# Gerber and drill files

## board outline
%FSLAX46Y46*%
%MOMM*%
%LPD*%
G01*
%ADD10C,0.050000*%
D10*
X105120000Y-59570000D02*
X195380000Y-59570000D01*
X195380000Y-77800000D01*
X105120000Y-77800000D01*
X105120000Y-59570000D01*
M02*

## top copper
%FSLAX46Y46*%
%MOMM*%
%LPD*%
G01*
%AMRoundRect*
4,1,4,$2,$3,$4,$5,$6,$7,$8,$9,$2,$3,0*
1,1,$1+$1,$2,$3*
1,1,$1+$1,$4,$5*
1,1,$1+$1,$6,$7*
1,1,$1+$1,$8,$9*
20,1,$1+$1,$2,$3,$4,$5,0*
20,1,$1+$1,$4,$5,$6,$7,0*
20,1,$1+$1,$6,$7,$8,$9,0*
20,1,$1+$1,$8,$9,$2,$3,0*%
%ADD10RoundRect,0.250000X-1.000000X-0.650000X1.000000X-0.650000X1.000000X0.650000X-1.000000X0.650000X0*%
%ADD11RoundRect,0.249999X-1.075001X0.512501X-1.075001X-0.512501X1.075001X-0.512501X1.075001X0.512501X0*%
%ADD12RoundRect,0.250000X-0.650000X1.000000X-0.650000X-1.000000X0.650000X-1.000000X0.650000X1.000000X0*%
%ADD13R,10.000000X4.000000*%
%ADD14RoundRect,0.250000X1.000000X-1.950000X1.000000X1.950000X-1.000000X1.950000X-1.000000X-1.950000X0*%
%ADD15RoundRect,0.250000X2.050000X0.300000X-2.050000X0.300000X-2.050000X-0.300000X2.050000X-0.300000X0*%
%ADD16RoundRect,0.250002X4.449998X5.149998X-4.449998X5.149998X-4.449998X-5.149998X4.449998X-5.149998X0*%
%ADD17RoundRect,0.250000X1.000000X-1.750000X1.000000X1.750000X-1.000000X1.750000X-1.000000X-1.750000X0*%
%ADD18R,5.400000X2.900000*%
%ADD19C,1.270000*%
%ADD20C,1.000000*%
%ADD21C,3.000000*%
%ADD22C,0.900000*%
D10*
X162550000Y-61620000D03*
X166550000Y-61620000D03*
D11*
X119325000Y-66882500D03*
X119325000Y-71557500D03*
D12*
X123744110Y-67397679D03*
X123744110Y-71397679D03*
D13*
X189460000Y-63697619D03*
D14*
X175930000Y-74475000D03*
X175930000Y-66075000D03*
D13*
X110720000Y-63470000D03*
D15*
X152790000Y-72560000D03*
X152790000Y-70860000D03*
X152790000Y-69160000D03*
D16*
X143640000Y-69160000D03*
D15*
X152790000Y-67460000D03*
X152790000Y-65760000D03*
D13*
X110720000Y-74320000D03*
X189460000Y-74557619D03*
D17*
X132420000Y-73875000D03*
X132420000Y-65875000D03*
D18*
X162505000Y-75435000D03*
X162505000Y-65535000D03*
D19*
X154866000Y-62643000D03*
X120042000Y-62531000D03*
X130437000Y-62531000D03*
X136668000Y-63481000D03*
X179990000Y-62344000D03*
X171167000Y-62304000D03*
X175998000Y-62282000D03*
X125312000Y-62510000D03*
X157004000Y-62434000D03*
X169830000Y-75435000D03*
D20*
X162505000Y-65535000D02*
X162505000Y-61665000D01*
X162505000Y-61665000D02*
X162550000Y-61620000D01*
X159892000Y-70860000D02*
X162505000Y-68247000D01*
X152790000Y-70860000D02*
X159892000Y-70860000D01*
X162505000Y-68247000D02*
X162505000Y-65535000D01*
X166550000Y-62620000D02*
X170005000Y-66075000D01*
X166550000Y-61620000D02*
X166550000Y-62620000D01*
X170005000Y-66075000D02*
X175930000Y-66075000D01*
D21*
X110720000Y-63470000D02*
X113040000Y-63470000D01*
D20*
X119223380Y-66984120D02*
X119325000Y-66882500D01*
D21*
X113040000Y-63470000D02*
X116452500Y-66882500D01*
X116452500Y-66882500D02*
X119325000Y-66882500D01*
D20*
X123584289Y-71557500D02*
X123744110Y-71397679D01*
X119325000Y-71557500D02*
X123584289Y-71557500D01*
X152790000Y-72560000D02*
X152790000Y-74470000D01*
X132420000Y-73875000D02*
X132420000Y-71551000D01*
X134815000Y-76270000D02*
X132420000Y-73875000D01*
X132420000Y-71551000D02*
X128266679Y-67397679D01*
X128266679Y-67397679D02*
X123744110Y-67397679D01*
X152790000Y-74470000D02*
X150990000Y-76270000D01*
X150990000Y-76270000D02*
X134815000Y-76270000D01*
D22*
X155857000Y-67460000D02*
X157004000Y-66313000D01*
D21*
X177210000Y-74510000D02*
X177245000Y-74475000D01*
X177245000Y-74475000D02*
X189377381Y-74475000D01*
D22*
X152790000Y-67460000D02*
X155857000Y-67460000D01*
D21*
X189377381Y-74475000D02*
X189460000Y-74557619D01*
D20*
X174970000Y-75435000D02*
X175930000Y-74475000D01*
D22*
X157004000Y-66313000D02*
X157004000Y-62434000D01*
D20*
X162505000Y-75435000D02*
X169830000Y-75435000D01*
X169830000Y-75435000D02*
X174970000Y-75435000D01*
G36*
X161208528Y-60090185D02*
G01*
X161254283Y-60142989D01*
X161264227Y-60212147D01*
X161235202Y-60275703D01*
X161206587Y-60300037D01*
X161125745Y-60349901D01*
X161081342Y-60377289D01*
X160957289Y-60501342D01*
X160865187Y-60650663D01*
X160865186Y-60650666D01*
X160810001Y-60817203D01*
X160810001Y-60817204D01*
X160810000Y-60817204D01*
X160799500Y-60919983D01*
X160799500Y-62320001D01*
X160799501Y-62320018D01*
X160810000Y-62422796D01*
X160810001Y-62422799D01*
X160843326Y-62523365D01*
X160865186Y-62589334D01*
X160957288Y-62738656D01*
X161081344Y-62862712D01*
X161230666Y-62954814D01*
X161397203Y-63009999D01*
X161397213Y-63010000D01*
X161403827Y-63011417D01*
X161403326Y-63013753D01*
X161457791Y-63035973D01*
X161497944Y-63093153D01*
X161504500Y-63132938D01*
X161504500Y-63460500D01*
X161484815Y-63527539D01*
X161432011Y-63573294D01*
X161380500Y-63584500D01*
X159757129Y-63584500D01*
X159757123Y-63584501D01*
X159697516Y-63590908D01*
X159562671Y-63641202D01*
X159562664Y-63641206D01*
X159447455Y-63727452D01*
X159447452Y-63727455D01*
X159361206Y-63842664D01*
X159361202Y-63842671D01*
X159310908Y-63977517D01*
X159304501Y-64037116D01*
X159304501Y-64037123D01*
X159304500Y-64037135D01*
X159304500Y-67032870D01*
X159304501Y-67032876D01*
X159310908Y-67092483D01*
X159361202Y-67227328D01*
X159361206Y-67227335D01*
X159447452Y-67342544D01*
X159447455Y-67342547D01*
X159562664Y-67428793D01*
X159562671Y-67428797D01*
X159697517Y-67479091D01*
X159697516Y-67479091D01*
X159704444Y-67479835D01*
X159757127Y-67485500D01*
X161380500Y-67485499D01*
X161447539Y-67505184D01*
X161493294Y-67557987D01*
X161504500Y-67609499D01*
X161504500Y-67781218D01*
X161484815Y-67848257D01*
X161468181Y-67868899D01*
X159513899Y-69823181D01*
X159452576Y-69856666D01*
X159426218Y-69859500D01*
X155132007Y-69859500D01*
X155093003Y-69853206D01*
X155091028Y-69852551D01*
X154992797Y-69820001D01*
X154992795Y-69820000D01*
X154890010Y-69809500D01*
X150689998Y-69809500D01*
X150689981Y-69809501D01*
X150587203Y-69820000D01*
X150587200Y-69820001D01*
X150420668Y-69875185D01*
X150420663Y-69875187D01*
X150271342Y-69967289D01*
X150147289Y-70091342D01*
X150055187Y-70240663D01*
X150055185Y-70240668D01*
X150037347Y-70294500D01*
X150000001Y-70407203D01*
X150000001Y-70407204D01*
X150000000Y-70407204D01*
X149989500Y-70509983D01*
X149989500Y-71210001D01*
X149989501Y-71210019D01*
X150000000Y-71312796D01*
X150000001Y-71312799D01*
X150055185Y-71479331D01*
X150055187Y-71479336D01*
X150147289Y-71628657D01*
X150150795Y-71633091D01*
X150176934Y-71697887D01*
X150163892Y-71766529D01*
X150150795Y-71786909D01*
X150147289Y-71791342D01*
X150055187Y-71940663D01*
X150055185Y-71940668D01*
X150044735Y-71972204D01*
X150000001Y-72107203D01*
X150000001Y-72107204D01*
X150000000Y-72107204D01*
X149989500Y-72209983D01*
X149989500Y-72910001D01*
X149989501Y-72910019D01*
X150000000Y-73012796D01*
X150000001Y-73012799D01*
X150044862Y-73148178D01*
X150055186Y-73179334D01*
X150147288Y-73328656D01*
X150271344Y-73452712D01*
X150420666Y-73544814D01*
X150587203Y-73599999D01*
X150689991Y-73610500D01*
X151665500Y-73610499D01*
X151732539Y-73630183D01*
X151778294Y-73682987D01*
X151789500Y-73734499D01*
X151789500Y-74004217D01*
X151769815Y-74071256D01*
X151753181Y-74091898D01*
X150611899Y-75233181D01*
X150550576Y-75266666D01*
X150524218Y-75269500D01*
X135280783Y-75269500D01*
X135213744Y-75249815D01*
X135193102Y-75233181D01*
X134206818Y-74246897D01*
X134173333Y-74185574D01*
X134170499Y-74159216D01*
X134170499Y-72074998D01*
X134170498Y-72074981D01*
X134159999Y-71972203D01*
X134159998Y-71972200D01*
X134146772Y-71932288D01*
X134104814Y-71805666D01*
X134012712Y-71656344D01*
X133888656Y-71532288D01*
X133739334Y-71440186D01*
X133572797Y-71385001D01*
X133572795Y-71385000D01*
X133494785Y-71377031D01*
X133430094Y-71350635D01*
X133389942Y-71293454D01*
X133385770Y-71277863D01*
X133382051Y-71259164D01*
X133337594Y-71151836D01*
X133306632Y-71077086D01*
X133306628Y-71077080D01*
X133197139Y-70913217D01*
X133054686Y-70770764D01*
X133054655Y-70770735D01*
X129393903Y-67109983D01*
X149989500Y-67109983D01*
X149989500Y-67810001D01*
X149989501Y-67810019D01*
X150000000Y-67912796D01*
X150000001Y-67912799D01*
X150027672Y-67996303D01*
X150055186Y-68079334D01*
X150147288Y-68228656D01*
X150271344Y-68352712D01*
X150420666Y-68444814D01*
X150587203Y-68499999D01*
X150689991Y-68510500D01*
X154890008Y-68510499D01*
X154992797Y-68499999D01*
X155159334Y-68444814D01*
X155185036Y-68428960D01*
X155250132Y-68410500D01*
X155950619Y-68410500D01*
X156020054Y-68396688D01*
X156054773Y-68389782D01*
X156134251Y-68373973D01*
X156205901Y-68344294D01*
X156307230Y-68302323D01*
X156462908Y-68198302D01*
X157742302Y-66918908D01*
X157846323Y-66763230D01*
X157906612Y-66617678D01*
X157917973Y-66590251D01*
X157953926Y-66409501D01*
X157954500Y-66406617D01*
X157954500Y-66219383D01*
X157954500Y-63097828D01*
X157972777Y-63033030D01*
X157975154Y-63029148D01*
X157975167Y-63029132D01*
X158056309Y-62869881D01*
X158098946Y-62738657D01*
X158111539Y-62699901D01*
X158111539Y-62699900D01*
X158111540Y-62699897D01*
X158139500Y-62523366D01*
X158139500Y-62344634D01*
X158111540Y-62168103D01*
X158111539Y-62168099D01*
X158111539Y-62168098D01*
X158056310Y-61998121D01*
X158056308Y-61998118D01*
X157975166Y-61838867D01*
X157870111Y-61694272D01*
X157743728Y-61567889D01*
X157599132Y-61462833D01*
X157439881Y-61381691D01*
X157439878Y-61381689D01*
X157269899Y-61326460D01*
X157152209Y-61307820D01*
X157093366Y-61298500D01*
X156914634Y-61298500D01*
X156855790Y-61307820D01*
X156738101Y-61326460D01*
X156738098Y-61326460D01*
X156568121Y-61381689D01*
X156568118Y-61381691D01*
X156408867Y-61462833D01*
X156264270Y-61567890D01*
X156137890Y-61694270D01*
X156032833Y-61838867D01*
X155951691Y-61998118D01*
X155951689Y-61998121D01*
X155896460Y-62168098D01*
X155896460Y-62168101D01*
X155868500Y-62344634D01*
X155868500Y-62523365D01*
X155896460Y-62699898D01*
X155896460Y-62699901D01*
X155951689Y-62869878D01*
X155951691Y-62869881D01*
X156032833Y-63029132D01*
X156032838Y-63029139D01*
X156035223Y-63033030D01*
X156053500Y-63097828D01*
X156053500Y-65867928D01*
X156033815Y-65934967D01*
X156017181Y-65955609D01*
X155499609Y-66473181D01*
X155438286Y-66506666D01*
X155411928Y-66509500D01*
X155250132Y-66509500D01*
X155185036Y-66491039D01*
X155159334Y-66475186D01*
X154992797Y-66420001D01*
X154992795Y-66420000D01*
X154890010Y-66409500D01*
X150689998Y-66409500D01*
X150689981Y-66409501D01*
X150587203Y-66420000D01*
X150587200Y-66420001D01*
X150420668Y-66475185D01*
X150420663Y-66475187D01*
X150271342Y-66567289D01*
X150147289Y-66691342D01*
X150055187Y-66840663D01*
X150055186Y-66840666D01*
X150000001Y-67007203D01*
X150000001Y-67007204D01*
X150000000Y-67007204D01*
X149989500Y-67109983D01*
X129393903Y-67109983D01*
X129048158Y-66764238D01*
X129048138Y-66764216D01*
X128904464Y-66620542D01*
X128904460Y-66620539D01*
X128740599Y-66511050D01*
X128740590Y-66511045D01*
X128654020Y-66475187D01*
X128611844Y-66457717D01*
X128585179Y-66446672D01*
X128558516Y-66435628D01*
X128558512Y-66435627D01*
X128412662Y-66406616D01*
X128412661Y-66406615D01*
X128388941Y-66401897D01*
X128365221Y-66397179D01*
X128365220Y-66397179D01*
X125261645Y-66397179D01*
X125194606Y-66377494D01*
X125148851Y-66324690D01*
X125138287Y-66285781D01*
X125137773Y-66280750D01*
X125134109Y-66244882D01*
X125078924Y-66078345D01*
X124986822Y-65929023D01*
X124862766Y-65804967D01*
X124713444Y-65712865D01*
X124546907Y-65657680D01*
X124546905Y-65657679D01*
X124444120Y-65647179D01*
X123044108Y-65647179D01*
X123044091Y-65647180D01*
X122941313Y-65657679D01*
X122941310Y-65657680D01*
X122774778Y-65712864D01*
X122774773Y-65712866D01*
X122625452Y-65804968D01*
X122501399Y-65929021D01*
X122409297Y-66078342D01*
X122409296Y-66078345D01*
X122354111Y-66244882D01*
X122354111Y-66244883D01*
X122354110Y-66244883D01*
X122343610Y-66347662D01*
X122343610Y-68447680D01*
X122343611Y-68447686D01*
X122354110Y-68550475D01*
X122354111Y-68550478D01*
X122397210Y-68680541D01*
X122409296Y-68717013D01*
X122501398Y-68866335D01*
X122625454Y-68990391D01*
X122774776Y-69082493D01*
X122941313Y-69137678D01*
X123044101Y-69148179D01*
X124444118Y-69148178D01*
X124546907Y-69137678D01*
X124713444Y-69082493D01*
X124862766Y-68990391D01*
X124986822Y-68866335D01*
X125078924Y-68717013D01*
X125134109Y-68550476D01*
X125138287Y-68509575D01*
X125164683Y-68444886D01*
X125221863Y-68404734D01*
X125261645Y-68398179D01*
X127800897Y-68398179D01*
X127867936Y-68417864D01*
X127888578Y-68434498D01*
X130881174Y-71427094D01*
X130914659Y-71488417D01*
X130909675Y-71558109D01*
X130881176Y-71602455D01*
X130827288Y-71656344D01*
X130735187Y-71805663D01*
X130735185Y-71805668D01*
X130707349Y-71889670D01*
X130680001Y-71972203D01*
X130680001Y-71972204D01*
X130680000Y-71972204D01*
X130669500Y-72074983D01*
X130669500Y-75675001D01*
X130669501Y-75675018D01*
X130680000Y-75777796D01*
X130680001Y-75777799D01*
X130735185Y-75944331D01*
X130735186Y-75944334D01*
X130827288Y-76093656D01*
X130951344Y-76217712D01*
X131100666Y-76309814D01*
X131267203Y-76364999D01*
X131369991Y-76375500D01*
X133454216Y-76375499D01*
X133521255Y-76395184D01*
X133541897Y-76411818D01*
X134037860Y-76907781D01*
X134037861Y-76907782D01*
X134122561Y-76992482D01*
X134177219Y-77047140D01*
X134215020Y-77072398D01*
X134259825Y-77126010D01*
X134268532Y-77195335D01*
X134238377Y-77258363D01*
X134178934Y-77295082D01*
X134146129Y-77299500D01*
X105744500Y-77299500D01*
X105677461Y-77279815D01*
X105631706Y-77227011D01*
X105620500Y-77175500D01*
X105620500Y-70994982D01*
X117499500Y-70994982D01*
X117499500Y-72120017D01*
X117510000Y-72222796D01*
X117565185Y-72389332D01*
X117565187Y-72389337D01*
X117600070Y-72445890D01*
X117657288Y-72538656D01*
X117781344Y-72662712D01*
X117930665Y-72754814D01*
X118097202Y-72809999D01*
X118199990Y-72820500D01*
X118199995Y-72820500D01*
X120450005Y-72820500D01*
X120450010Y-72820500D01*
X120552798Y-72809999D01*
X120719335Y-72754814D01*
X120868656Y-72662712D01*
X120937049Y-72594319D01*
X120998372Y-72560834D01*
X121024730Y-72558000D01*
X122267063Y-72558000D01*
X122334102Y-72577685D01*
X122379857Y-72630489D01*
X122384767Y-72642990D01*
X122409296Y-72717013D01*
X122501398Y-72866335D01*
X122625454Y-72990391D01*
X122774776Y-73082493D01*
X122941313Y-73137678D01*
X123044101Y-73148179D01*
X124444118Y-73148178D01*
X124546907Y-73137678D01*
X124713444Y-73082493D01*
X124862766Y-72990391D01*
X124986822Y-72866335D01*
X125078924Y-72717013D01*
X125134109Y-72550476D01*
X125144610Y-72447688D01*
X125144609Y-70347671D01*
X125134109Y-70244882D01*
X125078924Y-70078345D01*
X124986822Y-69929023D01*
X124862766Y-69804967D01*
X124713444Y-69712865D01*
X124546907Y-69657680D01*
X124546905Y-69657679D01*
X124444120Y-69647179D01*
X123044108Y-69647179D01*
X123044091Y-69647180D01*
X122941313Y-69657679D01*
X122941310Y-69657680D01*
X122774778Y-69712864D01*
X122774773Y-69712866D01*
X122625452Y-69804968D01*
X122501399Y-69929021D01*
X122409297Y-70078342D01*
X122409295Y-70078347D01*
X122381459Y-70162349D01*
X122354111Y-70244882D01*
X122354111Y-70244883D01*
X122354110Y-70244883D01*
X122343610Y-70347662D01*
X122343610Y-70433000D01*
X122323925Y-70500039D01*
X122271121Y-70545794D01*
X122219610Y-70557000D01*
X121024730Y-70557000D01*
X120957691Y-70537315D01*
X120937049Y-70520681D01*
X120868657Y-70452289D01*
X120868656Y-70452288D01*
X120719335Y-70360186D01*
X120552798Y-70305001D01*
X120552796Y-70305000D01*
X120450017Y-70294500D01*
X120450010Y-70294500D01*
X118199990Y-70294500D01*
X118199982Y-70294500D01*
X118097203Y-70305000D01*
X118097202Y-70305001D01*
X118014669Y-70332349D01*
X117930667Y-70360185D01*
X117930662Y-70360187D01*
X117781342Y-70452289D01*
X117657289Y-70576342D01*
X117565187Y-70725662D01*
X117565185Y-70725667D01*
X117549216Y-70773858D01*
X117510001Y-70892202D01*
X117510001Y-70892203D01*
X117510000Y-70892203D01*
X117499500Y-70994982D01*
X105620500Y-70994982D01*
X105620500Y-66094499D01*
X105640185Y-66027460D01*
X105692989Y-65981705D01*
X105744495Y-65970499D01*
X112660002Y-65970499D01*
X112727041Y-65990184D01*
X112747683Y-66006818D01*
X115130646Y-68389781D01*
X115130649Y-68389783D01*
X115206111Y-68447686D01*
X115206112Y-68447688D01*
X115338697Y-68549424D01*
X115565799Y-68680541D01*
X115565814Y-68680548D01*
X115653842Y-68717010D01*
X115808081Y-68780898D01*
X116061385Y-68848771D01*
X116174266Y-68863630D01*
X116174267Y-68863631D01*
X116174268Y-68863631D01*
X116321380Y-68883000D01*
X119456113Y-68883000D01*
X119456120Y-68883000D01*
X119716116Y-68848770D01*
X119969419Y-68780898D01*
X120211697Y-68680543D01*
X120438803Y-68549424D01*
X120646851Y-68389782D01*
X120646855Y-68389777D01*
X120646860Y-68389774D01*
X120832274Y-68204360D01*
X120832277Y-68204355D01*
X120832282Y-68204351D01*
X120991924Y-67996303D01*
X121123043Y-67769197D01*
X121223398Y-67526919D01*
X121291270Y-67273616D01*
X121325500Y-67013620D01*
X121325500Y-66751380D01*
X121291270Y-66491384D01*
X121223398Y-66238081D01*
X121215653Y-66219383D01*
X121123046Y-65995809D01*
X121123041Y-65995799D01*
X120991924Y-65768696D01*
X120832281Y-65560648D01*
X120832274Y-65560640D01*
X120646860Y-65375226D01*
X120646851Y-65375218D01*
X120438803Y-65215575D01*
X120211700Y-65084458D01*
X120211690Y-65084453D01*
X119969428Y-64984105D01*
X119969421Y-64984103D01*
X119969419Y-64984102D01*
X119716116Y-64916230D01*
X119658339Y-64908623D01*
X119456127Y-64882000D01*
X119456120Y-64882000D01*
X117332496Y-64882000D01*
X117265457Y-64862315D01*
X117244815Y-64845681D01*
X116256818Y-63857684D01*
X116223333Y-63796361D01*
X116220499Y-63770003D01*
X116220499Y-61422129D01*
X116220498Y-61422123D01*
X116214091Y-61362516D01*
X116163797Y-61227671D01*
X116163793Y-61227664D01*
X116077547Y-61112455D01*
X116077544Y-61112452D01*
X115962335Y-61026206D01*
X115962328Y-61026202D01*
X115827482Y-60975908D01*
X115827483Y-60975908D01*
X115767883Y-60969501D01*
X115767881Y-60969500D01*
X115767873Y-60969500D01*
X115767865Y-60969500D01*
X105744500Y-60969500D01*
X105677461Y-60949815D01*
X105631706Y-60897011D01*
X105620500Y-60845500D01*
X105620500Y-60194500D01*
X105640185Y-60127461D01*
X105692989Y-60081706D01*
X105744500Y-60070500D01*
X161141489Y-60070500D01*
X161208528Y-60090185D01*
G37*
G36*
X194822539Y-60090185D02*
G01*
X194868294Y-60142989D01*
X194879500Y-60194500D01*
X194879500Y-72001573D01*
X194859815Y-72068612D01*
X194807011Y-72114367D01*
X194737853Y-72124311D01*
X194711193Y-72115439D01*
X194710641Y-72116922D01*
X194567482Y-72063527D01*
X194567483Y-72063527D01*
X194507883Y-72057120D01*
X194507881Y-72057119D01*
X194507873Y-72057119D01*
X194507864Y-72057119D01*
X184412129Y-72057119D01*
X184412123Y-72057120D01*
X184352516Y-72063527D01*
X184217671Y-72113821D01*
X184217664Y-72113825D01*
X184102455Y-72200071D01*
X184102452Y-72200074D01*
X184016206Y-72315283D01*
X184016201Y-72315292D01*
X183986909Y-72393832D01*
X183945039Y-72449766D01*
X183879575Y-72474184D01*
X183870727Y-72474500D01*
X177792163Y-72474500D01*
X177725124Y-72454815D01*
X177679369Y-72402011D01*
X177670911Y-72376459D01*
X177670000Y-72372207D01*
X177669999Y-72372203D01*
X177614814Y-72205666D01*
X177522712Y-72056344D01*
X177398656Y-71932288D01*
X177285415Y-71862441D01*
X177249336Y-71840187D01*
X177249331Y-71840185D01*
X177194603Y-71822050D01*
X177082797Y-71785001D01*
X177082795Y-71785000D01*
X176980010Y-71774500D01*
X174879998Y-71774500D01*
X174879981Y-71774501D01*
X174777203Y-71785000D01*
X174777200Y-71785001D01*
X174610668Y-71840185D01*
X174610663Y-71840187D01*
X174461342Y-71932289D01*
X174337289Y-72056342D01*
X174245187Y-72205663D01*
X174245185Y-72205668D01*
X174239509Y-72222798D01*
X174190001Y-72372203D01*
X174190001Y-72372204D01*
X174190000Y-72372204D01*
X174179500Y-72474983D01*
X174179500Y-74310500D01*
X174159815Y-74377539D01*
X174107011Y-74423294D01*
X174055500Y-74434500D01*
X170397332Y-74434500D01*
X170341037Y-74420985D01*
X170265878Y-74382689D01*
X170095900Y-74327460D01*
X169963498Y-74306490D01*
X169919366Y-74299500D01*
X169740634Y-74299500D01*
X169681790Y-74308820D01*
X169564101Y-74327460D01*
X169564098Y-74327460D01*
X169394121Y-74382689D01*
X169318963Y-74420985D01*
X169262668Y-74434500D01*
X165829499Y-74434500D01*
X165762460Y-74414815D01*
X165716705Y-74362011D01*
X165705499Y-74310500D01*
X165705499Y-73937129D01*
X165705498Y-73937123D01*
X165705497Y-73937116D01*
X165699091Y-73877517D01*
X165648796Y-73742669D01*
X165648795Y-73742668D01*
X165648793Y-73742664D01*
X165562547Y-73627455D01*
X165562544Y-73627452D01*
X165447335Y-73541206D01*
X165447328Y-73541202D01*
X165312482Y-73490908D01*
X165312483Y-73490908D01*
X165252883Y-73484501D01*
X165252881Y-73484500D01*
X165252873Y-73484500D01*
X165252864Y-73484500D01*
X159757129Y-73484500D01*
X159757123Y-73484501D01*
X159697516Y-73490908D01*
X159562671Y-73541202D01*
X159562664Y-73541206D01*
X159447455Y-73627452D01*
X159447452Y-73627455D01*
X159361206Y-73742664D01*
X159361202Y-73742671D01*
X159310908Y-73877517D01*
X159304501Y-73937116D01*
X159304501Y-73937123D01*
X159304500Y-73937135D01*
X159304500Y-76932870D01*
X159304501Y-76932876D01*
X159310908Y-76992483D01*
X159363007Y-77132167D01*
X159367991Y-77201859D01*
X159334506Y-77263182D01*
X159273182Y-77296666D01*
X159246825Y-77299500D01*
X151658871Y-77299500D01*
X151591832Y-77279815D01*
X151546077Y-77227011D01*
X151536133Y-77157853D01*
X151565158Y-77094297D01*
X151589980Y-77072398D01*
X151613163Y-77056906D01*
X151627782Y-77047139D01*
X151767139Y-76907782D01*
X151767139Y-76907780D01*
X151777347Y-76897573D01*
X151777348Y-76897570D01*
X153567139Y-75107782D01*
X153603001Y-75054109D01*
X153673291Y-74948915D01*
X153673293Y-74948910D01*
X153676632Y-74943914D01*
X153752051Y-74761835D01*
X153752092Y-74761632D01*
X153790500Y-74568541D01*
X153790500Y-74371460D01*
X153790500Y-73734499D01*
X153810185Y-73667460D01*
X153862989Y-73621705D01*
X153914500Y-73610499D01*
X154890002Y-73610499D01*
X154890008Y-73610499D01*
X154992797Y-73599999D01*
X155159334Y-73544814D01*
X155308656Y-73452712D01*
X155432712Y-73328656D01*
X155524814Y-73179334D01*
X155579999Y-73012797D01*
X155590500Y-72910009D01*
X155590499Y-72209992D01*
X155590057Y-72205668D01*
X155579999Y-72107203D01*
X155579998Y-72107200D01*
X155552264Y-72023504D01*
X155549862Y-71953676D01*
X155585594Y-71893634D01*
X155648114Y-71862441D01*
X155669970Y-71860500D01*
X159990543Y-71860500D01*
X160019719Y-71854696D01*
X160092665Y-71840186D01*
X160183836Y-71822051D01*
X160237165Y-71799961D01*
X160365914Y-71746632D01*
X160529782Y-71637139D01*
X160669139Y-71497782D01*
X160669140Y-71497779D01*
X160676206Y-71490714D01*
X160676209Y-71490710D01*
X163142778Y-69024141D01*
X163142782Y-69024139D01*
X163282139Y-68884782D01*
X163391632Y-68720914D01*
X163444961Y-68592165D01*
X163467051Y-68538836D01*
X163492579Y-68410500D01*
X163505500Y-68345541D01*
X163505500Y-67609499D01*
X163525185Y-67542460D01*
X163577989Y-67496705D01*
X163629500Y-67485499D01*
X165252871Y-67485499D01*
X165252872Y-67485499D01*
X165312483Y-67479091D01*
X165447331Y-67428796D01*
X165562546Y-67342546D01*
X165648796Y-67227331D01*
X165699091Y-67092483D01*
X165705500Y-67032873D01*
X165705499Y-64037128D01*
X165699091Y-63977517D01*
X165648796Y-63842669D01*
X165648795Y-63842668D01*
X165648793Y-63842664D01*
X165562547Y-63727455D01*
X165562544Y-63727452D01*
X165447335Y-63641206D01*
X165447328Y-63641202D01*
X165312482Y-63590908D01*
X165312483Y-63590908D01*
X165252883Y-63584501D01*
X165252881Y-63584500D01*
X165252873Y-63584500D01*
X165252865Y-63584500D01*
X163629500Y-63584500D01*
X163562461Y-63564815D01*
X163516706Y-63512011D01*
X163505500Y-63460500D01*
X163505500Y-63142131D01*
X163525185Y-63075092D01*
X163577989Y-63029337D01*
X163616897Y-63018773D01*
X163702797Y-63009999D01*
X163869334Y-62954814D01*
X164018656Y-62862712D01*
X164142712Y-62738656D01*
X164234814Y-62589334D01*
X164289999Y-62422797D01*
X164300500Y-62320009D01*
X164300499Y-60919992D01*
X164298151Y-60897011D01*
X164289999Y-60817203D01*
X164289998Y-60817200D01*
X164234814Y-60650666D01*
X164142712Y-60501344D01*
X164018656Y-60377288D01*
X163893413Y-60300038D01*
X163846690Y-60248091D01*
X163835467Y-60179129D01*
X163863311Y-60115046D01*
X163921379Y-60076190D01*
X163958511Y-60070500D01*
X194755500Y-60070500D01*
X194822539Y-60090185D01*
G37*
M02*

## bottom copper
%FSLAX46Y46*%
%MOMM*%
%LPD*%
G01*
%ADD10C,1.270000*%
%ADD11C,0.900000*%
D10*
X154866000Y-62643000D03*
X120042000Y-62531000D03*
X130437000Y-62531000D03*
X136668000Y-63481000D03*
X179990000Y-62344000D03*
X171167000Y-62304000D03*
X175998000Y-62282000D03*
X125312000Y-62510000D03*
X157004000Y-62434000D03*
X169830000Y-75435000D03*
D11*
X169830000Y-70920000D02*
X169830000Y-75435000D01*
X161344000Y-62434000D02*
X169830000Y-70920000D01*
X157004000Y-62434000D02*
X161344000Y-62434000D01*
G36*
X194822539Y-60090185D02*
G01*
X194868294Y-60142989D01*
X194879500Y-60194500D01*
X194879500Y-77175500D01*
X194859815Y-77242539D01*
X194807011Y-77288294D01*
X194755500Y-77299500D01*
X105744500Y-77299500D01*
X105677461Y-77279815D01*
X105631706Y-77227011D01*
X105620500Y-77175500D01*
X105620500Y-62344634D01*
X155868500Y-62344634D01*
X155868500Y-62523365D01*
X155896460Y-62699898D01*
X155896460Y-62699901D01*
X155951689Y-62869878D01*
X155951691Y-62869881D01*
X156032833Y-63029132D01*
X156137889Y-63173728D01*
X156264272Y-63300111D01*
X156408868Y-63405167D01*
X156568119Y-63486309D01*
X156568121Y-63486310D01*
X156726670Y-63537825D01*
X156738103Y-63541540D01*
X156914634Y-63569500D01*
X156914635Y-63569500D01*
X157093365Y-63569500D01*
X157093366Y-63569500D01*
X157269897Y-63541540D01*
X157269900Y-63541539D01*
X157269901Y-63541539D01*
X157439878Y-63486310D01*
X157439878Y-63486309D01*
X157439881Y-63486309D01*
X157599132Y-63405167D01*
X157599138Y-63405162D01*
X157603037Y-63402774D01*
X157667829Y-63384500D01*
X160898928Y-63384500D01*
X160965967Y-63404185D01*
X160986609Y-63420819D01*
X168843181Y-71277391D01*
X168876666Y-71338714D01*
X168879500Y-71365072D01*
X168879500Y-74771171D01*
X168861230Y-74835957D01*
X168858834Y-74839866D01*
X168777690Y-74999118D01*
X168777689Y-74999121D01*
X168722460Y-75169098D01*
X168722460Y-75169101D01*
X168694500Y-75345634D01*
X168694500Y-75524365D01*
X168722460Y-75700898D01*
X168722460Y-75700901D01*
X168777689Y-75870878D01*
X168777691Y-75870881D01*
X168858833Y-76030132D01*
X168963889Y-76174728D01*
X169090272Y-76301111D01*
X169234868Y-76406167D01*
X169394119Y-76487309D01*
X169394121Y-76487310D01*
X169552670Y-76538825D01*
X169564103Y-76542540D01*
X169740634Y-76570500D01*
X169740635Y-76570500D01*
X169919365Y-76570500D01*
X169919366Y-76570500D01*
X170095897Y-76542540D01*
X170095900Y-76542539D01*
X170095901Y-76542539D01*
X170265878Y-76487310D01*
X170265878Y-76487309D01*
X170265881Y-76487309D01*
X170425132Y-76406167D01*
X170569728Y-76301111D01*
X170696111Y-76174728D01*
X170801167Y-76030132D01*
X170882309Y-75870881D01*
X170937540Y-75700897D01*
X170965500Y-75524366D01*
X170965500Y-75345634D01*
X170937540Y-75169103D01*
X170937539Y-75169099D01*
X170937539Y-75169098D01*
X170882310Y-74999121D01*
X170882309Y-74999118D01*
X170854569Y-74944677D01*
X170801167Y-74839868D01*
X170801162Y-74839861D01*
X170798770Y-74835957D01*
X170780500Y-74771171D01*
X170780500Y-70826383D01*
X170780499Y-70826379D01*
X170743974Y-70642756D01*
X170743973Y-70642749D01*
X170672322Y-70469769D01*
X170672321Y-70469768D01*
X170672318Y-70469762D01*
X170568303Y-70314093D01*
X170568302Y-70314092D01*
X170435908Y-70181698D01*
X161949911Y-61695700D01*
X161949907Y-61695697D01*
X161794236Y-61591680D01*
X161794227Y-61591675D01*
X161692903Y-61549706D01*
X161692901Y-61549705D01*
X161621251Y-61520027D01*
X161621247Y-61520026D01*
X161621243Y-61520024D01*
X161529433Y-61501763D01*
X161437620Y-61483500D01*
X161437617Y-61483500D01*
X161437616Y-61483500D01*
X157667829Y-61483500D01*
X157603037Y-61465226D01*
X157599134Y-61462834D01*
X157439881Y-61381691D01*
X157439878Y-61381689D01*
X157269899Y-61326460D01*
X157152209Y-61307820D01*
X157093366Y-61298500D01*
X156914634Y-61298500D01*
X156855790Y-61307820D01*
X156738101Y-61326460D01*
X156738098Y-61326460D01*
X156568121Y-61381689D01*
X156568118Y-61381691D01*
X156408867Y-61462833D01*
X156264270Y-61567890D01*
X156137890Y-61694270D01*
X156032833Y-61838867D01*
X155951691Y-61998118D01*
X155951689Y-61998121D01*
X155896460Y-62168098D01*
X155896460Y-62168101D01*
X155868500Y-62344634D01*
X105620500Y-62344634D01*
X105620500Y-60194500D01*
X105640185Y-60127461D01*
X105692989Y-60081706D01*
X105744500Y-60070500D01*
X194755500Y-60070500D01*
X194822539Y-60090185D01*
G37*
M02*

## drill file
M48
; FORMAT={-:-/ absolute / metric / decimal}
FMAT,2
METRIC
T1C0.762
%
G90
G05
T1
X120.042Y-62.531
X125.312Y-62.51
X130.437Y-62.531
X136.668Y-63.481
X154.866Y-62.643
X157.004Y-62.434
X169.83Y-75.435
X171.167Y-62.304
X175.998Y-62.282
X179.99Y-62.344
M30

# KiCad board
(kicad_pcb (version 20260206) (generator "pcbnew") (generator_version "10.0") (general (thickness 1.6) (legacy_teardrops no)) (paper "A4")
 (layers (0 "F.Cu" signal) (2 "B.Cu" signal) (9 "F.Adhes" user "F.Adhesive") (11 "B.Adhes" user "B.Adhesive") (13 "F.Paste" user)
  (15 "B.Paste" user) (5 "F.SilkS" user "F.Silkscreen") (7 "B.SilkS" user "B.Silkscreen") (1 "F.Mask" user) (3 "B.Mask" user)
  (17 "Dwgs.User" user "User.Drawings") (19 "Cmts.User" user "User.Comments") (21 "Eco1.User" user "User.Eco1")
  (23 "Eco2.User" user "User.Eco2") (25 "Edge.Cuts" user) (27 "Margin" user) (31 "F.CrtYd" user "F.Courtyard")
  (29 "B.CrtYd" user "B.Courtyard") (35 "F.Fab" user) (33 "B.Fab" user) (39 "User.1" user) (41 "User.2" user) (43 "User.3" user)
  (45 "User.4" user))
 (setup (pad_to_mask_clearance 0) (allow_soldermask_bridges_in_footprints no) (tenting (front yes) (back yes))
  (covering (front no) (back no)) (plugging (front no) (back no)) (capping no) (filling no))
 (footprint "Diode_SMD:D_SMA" (layer "F.Cu") (at 164.55 61.62)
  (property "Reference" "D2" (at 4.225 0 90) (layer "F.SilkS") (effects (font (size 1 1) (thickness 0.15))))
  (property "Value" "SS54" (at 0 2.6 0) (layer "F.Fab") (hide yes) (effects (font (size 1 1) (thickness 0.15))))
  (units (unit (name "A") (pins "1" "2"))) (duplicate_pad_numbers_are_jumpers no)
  (pad "1" smd roundrect (at -2 0) (size 2.5 1.8) (layers "F.Cu" "F.Mask" "F.Paste") (roundrect_rratio 0.1388888889) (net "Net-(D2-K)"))
  (pad "2" smd roundrect (at 2 0) (size 2.5 1.8) (layers "F.Cu" "F.Mask" "F.Paste") (roundrect_rratio 0.1388888889) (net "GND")))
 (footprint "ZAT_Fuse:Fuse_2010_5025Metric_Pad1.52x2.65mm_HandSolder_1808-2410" (layer "F.Cu") (at 119.325 69.22 -90)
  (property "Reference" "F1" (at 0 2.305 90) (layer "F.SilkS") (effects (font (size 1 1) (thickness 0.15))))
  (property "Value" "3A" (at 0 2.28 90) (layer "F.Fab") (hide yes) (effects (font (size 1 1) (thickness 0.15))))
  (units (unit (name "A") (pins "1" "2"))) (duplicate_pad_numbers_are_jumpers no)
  (pad "1" smd roundrect (at -2.3375 0 270) (size 1.525 2.65) (layers "F.Cu" "F.Mask" "F.Paste") (roundrect_rratio 0.163934) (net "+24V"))
  (pad "2" smd roundrect (at 2.3375 0 270) (size 1.525 2.65) (layers "F.Cu" "F.Mask" "F.Paste") (roundrect_rratio 0.163934)
   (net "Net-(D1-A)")))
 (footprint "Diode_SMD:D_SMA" (layer "F.Cu") (at 123.74411 69.397679 -90)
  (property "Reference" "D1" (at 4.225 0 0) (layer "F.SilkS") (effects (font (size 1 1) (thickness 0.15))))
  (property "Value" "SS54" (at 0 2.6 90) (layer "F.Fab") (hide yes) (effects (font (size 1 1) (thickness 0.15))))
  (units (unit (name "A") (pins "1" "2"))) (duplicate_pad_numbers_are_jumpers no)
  (pad "1" smd roundrect (at -2 0 270) (size 2.5 1.8) (layers "F.Cu" "F.Mask" "F.Paste") (roundrect_rratio 0.1388888889) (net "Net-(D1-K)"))
  (pad "2" smd roundrect (at 2 0 270) (size 2.5 1.8) (layers "F.Cu" "F.Mask" "F.Paste") (roundrect_rratio 0.1388888889) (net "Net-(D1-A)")))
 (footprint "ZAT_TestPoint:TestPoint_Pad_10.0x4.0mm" (layer "F.Cu") (at 189.46 63.697619)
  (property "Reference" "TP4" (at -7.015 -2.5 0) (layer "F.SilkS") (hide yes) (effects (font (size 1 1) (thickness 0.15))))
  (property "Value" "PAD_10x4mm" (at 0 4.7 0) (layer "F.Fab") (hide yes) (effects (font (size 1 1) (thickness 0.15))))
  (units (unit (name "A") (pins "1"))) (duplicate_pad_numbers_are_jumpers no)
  (pad "1" smd rect (at 0 0) (size 10 4) (layers "F.Cu" "F.Mask" "F.Paste") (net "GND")))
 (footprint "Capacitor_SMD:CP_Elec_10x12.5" (layer "F.Cu") (at 175.93 70.275 90)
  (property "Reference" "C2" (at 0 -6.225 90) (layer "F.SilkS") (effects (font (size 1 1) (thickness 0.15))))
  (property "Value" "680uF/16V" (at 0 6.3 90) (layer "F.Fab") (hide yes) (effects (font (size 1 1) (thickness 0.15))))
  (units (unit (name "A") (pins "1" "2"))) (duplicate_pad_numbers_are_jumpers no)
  (pad "1" smd roundrect (at -4.2 0 90) (size 4.4 2.5) (layers "F.Cu" "F.Mask" "F.Paste") (roundrect_rratio 0.1) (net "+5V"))
  (pad "2" smd roundrect (at 4.2 0 90) (size 4.4 2.5) (layers "F.Cu" "F.Mask" "F.Paste") (roundrect_rratio 0.1) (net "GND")))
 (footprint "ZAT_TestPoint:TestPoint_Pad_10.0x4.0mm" (layer "F.Cu") (at 110.72 63.47 180)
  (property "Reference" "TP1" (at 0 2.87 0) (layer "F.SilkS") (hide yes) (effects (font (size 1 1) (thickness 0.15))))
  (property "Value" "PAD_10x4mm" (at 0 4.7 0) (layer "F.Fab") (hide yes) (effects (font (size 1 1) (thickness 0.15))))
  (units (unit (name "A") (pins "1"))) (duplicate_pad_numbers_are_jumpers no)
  (pad "1" smd rect (at 0 0 180) (size 10 4) (layers "F.Cu" "F.Mask" "F.Paste") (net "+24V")))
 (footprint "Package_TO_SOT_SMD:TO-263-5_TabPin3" (layer "F.Cu") (at 145.14 69.16 180)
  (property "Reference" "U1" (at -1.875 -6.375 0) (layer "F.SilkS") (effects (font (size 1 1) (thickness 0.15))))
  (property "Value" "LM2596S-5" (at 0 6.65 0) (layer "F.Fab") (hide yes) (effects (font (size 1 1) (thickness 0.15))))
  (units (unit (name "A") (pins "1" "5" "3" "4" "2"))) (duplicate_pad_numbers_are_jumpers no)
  (pad "" smd roundrect (at -0.925 -2.775 180) (size 4.55 5.25) (layers "F.Paste") (roundrect_rratio 0.054945))
  (pad "" smd roundrect (at -0.925 2.775 180) (size 4.55 5.25) (layers "F.Paste") (roundrect_rratio 0.054945))
  (pad "" smd roundrect (at 3.925 -2.775 180) (size 4.55 5.25) (layers "F.Paste") (roundrect_rratio 0.054945))
  (pad "" smd roundrect (at 3.925 2.775 180) (size 4.55 5.25) (layers "F.Paste") (roundrect_rratio 0.054945))
  (pad "1" smd roundrect (at -7.65 -3.4 180) (size 4.6 1.1) (layers "F.Cu" "F.Mask" "F.Paste") (roundrect_rratio 0.227273)
   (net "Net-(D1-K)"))
  (pad "2" smd roundrect (at -7.65 -1.7 180) (size 4.6 1.1) (layers "F.Cu" "F.Mask" "F.Paste") (roundrect_rratio 0.227273)
   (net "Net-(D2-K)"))
  (pad "3" smd roundrect (at -7.65 0 180) (size 4.6 1.1) (layers "F.Cu" "F.Mask" "F.Paste") (roundrect_rratio 0.227273) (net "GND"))
  (pad "3" smd roundrect (at 1.5 0 180) (size 9.4 10.8) (layers "F.Cu" "F.Mask") (roundrect_rratio 0.026596) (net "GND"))
  (pad "4" smd roundrect (at -7.65 1.7 180) (size 4.6 1.1) (layers "F.Cu" "F.Mask" "F.Paste") (roundrect_rratio 0.227273) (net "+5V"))
  (pad "5" smd roundrect (at -7.65 3.4 180) (size 4.6 1.1) (layers "F.Cu" "F.Mask" "F.Paste") (roundrect_rratio 0.227273) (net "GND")))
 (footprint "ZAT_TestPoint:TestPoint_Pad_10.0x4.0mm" (layer "F.Cu") (at 110.72 74.32)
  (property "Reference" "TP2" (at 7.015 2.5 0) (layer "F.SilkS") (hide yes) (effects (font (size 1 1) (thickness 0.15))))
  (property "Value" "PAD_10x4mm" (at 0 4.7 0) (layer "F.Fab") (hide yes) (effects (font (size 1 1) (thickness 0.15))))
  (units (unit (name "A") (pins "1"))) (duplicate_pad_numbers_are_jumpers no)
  (pad "1" smd rect (at 0 0) (size 10 4) (layers "F.Cu" "F.Mask" "F.Paste") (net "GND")))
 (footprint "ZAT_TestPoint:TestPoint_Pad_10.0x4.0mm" (layer "F.Cu") (at 189.46 74.557619)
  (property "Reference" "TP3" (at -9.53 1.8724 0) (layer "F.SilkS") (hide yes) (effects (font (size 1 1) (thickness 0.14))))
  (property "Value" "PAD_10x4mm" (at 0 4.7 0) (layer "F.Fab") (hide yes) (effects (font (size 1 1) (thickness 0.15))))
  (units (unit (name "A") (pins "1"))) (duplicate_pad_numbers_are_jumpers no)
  (pad "1" smd rect (at 0 0) (size 10 4) (layers "F.Cu" "F.Mask" "F.Paste") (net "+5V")))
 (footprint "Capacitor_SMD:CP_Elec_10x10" (layer "F.Cu") (at 132.42 69.875 90)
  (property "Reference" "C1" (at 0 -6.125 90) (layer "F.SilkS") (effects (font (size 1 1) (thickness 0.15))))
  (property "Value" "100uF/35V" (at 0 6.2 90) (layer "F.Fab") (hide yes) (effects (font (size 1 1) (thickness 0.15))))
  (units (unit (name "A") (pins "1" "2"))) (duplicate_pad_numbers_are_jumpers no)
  (pad "1" smd roundrect (at -4 0 90) (size 4 2.5) (layers "F.Cu" "F.Mask" "F.Paste") (roundrect_rratio 0.1) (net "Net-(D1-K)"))
  (pad "2" smd roundrect (at 4 0 90) (size 4 2.5) (layers "F.Cu" "F.Mask" "F.Paste") (roundrect_rratio 0.1) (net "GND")))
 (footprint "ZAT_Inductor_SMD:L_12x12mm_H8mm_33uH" (layer "F.Cu") (at 162.505 70.485 90)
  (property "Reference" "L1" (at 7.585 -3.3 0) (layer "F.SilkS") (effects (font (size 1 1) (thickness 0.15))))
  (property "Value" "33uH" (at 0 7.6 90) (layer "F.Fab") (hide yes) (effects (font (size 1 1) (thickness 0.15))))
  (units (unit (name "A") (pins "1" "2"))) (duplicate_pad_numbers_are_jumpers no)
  (pad "1" smd rect (at -4.95 0 90) (size 2.9 5.4) (layers "F.Cu" "F.Mask" "F.Paste") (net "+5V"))
  (pad "2" smd rect (at 4.95 0 90) (size 2.9 5.4) (layers "F.Cu" "F.Mask" "F.Paste") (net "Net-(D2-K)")))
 (gr_rect (start 105.12 59.57) (end 195.38 77.8) (stroke (width 0.05) (type default)) (fill no) (layer "Edge.Cuts"))
 (segment (start 162.505 65.535) (end 162.505 61.665) (width 1) (layer "F.Cu") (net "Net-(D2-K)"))
 (segment (start 162.505 61.665) (end 162.55 61.62) (width 1) (layer "F.Cu") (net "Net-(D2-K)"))
 (segment (start 159.892 70.86) (end 162.505 68.247) (width 1) (layer "F.Cu") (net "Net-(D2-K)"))
 (segment (start 152.79 70.86) (end 159.892 70.86) (width 1) (layer "F.Cu") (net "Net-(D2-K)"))
 (segment (start 162.505 68.247) (end 162.505 65.535) (width 1) (layer "F.Cu") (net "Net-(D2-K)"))
 (segment (start 166.55 62.62) (end 170.005 66.075) (width 1) (layer "F.Cu") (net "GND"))
 (segment (start 166.55 61.62) (end 166.55 62.62) (width 1) (layer "F.Cu") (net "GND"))
 (segment (start 170.005 66.075) (end 175.93 66.075) (width 1) (layer "F.Cu") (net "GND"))
 (via (at 154.866 62.643) (size 1.27) (drill 0.762) (layers "F.Cu" "B.Cu") (free yes) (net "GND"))
 (via (at 120.042 62.531) (size 1.27) (drill 0.762) (layers "F.Cu" "B.Cu") (free yes) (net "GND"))
 (via (at 130.437 62.531) (size 1.27) (drill 0.762) (layers "F.Cu" "B.Cu") (free yes) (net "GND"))
 (via (at 136.668 63.481) (size 1.27) (drill 0.762) (layers "F.Cu" "B.Cu") (free yes) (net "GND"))
 (via (at 179.99 62.344) (size 1.27) (drill 0.762) (layers "F.Cu" "B.Cu") (free yes) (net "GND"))
 (via (at 171.167 62.304) (size 1.27) (drill 0.762) (layers "F.Cu" "B.Cu") (free yes) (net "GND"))
 (via (at 175.998 62.282) (size 1.27) (drill 0.762) (layers "F.Cu" "B.Cu") (free yes) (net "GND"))
 (via (at 125.312 62.51) (size 1.27) (drill 0.762) (layers "F.Cu" "B.Cu") (free yes) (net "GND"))
 (segment (start 110.72 63.47) (end 113.04 63.47) (width 3) (layer "F.Cu") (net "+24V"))
 (segment (start 119.22338 66.98412) (end 119.325 66.8825) (width 1) (layer "F.Cu") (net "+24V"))
 (segment (start 113.04 63.47) (end 116.4525 66.8825) (width 3) (layer "F.Cu") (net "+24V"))
 (segment (start 116.4525 66.8825) (end 119.325 66.8825) (width 3) (layer "F.Cu") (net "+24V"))
 (segment (start 123.584289 71.5575) (end 123.74411 71.397679) (width 1) (layer "F.Cu") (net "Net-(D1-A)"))
 (segment (start 119.325 71.5575) (end 123.584289 71.5575) (width 1) (layer "F.Cu") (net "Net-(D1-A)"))
 (segment (start 152.79 72.56) (end 152.79 74.47) (width 1) (layer "F.Cu") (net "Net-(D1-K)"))
 (segment (start 132.42 73.875) (end 132.42 71.551) (width 1) (layer "F.Cu") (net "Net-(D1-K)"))
 (segment (start 134.815 76.27) (end 132.42 73.875) (width 1) (layer "F.Cu") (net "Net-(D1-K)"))
 (segment (start 132.42 71.551) (end 128.266679 67.397679) (width 1) (layer "F.Cu") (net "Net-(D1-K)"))
 (segment (start 128.266679 67.397679) (end 123.74411 67.397679) (width 1) (layer "F.Cu") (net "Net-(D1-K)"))
 (segment (start 152.79 74.47) (end 150.99 76.27) (width 1) (layer "F.Cu") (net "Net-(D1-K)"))
 (segment (start 150.99 76.27) (end 134.815 76.27) (width 1) (layer "F.Cu") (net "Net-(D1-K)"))
 (segment (start 155.857 67.46) (end 157.004 66.313) (width 0.9) (layer "F.Cu") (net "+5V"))
 (segment (start 177.21 74.51) (end 177.245 74.475) (width 3) (layer "F.Cu") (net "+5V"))
 (segment (start 177.245 74.475) (end 189.377381 74.475) (width 3) (layer "F.Cu") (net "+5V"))
 (segment (start 152.79 67.46) (end 155.857 67.46) (width 0.9) (layer "F.Cu") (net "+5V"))
 (segment (start 189.377381 74.475) (end 189.46 74.557619) (width 3) (layer "F.Cu") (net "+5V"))
 (segment (start 174.97 75.435) (end 175.93 74.475) (width 1) (layer "F.Cu") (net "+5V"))
 (segment (start 157.004 66.313) (end 157.004 62.434) (width 0.9) (layer "F.Cu") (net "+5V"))
 (segment (start 162.505 75.435) (end 169.83 75.435) (width 1) (layer "F.Cu") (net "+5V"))
 (segment (start 169.83 75.435) (end 174.97 75.435) (width 1) (layer "F.Cu") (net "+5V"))
 (via (at 157.004 62.434) (size 1.27) (drill 0.762) (layers "F.Cu" "B.Cu") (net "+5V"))
 (via (at 169.83 75.435) (size 1.27) (drill 0.762) (layers "F.Cu" "B.Cu") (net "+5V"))
 (segment (start 169.83 70.92) (end 169.83 75.435) (width 0.9) (layer "B.Cu") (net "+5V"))
 (segment (start 161.344 62.434) (end 169.83 70.92) (width 0.9) (layer "B.Cu") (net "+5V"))
 (segment (start 157.004 62.434) (end 161.344 62.434) (width 0.9) (layer "B.Cu") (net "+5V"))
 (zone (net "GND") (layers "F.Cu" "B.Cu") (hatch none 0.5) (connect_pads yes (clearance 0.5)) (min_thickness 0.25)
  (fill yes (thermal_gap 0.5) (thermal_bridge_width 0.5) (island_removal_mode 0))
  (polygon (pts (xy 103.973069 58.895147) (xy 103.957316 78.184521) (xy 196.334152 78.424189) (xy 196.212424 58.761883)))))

